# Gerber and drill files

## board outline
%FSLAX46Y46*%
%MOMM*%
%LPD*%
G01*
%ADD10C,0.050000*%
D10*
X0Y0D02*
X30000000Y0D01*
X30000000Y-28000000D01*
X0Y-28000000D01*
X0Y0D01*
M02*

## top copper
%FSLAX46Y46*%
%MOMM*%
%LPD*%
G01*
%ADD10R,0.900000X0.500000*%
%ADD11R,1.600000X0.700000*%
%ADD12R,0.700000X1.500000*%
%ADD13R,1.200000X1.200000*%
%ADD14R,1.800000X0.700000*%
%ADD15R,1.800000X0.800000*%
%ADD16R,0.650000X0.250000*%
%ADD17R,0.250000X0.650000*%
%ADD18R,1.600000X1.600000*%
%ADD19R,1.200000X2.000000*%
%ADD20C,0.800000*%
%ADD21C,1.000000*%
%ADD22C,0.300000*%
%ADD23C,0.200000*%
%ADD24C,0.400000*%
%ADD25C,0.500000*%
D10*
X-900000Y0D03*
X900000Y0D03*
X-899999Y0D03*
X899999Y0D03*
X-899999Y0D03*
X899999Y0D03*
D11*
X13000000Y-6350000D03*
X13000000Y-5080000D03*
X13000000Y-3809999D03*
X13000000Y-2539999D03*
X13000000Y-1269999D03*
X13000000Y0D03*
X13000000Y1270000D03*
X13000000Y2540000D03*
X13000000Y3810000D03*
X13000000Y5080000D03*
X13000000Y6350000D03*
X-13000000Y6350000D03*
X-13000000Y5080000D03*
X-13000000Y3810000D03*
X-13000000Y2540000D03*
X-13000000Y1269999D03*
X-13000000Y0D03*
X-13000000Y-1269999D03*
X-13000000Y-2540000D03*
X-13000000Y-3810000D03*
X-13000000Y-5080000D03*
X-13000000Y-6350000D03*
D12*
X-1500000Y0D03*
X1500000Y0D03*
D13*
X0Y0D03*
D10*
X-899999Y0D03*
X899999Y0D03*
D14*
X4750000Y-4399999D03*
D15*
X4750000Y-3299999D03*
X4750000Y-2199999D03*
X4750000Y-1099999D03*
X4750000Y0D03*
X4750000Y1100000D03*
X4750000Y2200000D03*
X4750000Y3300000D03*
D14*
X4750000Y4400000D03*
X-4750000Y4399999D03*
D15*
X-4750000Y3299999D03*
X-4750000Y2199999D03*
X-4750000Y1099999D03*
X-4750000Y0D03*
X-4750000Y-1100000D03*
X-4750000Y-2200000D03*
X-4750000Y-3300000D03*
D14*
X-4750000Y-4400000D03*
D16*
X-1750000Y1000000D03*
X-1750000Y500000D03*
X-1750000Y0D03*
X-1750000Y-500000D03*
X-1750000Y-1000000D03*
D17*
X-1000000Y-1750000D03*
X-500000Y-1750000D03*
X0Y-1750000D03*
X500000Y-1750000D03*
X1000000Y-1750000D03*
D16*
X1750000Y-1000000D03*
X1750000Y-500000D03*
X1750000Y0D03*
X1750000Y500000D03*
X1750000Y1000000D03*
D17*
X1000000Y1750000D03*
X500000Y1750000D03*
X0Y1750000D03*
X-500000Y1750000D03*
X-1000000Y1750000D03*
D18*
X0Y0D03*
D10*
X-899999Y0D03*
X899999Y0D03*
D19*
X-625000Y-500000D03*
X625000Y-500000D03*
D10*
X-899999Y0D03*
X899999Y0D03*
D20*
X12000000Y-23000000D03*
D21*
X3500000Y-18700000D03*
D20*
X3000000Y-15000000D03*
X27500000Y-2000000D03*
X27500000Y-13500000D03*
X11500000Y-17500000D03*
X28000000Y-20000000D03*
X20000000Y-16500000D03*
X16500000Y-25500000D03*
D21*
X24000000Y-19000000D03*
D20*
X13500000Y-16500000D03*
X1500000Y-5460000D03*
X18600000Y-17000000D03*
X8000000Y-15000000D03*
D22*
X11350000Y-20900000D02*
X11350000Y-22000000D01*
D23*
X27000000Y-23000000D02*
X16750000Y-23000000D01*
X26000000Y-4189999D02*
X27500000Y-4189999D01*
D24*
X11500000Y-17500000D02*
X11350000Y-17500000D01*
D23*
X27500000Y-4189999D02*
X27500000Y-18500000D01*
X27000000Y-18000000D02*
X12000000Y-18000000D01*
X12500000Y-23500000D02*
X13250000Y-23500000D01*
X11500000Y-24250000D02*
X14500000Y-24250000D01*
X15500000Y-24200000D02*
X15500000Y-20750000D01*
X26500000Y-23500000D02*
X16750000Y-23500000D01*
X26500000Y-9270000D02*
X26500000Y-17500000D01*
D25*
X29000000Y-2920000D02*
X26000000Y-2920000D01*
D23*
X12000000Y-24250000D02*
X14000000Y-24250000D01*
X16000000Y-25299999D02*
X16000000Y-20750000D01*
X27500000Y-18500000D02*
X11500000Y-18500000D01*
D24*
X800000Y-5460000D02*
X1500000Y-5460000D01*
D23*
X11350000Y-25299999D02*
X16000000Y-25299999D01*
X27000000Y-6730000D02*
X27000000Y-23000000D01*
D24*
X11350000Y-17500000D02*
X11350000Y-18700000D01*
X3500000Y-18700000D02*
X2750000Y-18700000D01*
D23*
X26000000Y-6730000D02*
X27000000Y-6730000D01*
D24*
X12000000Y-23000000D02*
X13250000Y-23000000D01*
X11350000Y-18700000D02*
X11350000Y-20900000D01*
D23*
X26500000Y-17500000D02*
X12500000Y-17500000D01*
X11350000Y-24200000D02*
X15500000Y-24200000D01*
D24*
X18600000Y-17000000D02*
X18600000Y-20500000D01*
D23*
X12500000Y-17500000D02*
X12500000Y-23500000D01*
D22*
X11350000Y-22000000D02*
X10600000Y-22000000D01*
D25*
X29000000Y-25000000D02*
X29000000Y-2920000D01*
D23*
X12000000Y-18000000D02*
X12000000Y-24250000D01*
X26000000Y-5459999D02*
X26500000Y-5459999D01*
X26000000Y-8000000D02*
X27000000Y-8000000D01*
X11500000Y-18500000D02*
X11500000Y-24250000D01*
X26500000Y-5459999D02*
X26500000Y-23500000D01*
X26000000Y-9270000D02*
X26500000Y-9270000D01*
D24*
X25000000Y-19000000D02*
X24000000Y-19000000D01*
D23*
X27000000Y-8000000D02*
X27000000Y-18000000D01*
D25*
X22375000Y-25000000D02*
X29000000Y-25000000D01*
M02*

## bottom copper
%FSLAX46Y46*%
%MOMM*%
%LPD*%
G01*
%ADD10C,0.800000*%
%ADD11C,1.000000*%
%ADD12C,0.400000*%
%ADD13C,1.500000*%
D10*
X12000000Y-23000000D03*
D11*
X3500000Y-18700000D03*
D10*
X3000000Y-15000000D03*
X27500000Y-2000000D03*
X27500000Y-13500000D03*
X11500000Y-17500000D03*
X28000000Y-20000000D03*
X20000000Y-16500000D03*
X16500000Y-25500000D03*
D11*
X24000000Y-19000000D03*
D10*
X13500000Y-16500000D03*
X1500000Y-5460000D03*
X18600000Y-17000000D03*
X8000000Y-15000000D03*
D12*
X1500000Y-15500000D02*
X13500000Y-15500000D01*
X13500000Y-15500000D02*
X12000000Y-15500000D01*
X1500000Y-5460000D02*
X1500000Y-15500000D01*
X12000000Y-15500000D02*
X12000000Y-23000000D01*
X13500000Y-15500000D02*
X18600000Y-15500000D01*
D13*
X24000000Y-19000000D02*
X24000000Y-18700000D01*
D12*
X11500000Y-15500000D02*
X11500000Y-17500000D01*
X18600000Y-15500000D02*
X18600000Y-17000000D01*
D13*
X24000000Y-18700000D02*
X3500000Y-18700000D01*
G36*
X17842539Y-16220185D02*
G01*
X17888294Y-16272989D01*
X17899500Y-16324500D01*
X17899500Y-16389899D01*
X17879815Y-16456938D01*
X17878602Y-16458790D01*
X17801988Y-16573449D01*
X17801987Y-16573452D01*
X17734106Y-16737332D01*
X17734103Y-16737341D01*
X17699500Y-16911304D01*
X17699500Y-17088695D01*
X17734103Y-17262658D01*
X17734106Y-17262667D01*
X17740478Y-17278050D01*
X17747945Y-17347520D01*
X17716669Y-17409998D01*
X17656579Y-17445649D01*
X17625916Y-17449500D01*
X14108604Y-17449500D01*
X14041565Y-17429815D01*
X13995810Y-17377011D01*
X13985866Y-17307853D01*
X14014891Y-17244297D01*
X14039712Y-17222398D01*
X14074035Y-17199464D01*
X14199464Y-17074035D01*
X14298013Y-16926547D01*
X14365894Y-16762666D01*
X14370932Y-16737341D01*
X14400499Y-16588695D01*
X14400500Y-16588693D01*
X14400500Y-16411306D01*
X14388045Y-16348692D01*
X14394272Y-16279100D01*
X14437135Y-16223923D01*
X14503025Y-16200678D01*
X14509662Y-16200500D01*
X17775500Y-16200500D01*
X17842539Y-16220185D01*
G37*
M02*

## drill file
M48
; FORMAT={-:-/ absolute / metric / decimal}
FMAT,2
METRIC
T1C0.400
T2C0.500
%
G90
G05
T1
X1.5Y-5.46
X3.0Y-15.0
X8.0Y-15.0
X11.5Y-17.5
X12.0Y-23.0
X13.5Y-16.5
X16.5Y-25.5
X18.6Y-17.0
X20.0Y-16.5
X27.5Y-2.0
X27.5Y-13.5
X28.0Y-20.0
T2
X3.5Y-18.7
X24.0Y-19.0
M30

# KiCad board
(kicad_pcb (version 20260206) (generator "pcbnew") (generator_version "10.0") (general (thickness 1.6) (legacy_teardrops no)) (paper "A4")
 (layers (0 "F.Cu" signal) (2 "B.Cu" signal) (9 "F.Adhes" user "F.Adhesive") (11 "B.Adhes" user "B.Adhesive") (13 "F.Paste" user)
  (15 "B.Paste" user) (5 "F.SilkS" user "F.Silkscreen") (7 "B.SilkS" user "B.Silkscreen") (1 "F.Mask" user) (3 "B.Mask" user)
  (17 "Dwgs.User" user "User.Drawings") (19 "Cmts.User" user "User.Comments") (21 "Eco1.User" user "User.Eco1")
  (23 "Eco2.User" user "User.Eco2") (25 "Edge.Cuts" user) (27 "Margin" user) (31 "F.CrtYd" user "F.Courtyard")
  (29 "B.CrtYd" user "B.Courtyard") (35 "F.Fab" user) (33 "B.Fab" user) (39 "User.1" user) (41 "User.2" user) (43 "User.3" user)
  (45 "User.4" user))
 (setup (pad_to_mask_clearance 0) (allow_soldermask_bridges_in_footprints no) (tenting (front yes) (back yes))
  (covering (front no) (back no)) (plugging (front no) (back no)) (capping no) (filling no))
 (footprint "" (layer "F.Cu") (at 11.5 22)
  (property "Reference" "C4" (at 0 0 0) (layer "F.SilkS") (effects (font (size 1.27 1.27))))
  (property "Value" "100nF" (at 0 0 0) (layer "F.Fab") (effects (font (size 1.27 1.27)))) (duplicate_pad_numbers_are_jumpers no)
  (pad "1" smd rect (at -12.4 -22) (size 0.9 0.5) (layers "F.Cu" "F.Mask" "F.Paste") (thermal_bridge_angle 45))
  (pad "2" smd rect (at -10.6 -22) (size 0.9 0.5) (layers "F.Cu" "F.Mask" "F.Paste") (thermal_bridge_angle 45)))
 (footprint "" (layer "F.Cu") (at 27.5 5.5)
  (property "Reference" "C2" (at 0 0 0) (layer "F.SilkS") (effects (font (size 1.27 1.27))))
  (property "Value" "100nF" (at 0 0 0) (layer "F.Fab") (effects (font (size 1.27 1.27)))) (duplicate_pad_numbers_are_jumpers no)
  (pad "1" smd rect (at -28.399999 -5.5) (size 0.9 0.5) (layers "F.Cu" "F.Mask" "F.Paste") (thermal_bridge_angle 45))
  (pad "2" smd rect (at -26.600001 -5.5) (size 0.9 0.5) (layers "F.Cu" "F.Mask" "F.Paste") (thermal_bridge_angle 45)))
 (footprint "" (layer "F.Cu") (at 27.5 2.5)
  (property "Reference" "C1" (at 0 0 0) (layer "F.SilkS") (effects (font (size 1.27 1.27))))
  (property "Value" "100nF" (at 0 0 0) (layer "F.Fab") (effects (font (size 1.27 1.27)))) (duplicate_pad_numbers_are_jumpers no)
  (pad "1" smd rect (at -28.399999 -2.5) (size 0.9 0.5) (layers "F.Cu" "F.Mask" "F.Paste") (thermal_bridge_angle 45))
  (pad "2" smd rect (at -26.600001 -2.5) (size 0.9 0.5) (layers "F.Cu" "F.Mask" "F.Paste") (thermal_bridge_angle 45)))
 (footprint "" (layer "F.Cu") (at 13 8)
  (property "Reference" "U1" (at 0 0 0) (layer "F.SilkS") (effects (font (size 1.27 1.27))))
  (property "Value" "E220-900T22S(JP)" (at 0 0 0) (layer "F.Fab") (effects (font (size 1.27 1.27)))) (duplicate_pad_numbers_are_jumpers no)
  (pad "1" smd rect (at 0 -1.65) (size 1.6 0.7) (layers "F.Cu" "F.Mask" "F.Paste") (thermal_bridge_angle 45))
  (pad "2" smd rect (at 0 -2.92) (size 1.6 0.7) (layers "F.Cu" "F.Mask" "F.Paste") (thermal_bridge_angle 45))
  (pad "3" smd rect (at 0 -4.190001) (size 1.6 0.7) (layers "F.Cu" "F.Mask" "F.Paste") (thermal_bridge_angle 45))
  (pad "4" smd rect (at 0 -5.460001) (size 1.6 0.7) (layers "F.Cu" "F.Mask" "F.Paste") (thermal_bridge_angle 45))
  (pad "5" smd rect (at 0 -6.730001) (size 1.6 0.7) (layers "F.Cu" "F.Mask" "F.Paste") (thermal_bridge_angle 45))
  (pad "6" smd rect (at 0 -8) (size 1.6 0.7) (layers "F.Cu" "F.Mask" "F.Paste") (thermal_bridge_angle 45))
  (pad "7" smd rect (at 0 -9.27) (size 1.6 0.7) (layers "F.Cu" "F.Mask" "F.Paste") (thermal_bridge_angle 45))
  (pad "8" smd rect (at 0 -10.54) (size 1.6 0.7) (layers "F.Cu" "F.Mask" "F.Paste") (thermal_bridge_angle 45))
  (pad "9" smd rect (at 0 -11.81) (size 1.6 0.7) (layers "F.Cu" "F.Mask" "F.Paste") (thermal_bridge_angle 45))
  (pad "10" smd rect (at 0 -13.08) (size 1.6 0.7) (layers "F.Cu" "F.Mask" "F.Paste") (thermal_bridge_angle 45))
  (pad "11" smd rect (at 0 -14.35) (size 1.6 0.7) (layers "F.Cu" "F.Mask" "F.Paste") (thermal_bridge_angle 45))
  (pad "12" smd rect (at -26 -14.35) (size 1.6 0.7) (layers "F.Cu" "F.Mask" "F.Paste") (thermal_bridge_angle 45))
  (pad "13" smd rect (at -26 -13.08) (size 1.6 0.7) (layers "F.Cu" "F.Mask" "F.Paste") (thermal_bridge_angle 45))
  (pad "14" smd rect (at -26 -11.81) (size 1.6 0.7) (layers "F.Cu" "F.Mask" "F.Paste") (thermal_bridge_angle 45))
  (pad "15" smd rect (at -26 -10.54) (size 1.6 0.7) (layers "F.Cu" "F.Mask" "F.Paste") (thermal_bridge_angle 45))
  (pad "16" smd rect (at -26 -9.269999) (size 1.6 0.7) (layers "F.Cu" "F.Mask" "F.Paste") (thermal_bridge_angle 45))
  (pad "17" smd rect (at -26 -8) (size 1.6 0.7) (layers "F.Cu" "F.Mask" "F.Paste") (thermal_bridge_angle 45))
  (pad "18" smd rect (at -26 -6.730001) (size 1.6 0.7) (layers "F.Cu" "F.Mask" "F.Paste") (thermal_bridge_angle 45))
  (pad "19" smd rect (at -26 -5.46) (size 1.6 0.7) (layers "F.Cu" "F.Mask" "F.Paste") (thermal_bridge_angle 45))
  (pad "20" smd rect (at -26 -4.19) (size 1.6 0.7) (layers "F.Cu" "F.Mask" "F.Paste") (thermal_bridge_angle 45))
  (pad "21" smd rect (at -26 -2.92) (size 1.6 0.7) (layers "F.Cu" "F.Mask" "F.Paste") (thermal_bridge_angle 45))
  (pad "22" smd rect (at -26 -1.65) (size 1.6 0.7) (layers "F.Cu" "F.Mask" "F.Paste") (thermal_bridge_angle 45)))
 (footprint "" (layer "F.Cu") (at 25 19)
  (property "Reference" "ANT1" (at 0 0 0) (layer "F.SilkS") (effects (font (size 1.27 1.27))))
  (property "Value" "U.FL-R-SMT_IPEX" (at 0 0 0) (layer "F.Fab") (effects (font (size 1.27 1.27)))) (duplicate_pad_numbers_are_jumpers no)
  (pad "G1" smd rect (at -26.5 -19) (size 0.7 1.5) (layers "F.Cu" "F.Mask" "F.Paste") (thermal_bridge_angle 45))
  (pad "G2" smd rect (at -23.5 -19) (size 0.7 1.5) (layers "F.Cu" "F.Mask" "F.Paste") (thermal_bridge_angle 45))
  (pad "S" smd rect (at -25 -19) (size 1.2 1.2) (layers "F.Cu" "F.Mask" "F.Paste") (thermal_bridge_angle 45)))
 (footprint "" (layer "F.Cu") (at 19.5 24.5)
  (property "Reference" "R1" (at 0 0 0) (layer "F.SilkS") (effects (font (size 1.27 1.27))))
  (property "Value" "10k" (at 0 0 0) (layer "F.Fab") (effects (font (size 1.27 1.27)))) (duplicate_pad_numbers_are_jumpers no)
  (pad "1" smd rect (at -20.399999 -24.5) (size 0.9 0.5) (layers "F.Cu" "F.Mask" "F.Paste") (thermal_bridge_angle 45))
  (pad "2" smd rect (at -18.600001 -24.5) (size 0.9 0.5) (layers "F.Cu" "F.Mask" "F.Paste") (thermal_bridge_angle 45)))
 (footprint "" (layer "F.Cu") (at 6.6 22)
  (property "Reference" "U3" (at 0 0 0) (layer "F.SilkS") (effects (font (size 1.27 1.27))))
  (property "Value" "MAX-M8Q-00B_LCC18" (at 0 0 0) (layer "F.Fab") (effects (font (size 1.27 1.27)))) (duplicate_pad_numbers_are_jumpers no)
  (pad "1" smd rect (at -1.85 -17.600001) (size 1.8 0.7) (layers "F.Cu" "F.Mask" "F.Paste") (thermal_bridge_angle 45))
  (pad "2" smd rect (at -1.85 -18.700001) (size 1.8 0.8) (layers "F.Cu" "F.Mask" "F.Paste") (thermal_bridge_angle 45))
  (pad "3" smd rect (at -1.85 -19.800001) (size 1.8 0.8) (layers "F.Cu" "F.Mask" "F.Paste") (thermal_bridge_angle 45))
  (pad "4" smd rect (at -1.85 -20.900001) (size 1.8 0.8) (layers "F.Cu" "F.Mask" "F.Paste") (thermal_bridge_angle 45))
  (pad "5" smd rect (at -1.85 -22) (size 1.8 0.8) (layers "F.Cu" "F.Mask" "F.Paste") (thermal_bridge_angle 45))
  (pad "6" smd rect (at -1.85 -23.1) (size 1.8 0.8) (layers "F.Cu" "F.Mask" "F.Paste") (thermal_bridge_angle 45))
  (pad "7" smd rect (at -1.85 -24.2) (size 1.8 0.8) (layers "F.Cu" "F.Mask" "F.Paste") (thermal_bridge_angle 45))
  (pad "8" smd rect (at -1.85 -25.3) (size 1.8 0.8) (layers "F.Cu" "F.Mask" "F.Paste") (thermal_bridge_angle 45))
  (pad "9" smd rect (at -1.85 -26.4) (size 1.8 0.7) (layers "F.Cu" "F.Mask" "F.Paste") (thermal_bridge_angle 45))
  (pad "10" smd rect (at -11.35 -26.399999) (size 1.8 0.7) (layers "F.Cu" "F.Mask" "F.Paste") (thermal_bridge_angle 45))
  (pad "11" smd rect (at -11.35 -25.299999) (size 1.8 0.8) (layers "F.Cu" "F.Mask" "F.Paste") (thermal_bridge_angle 45))
  (pad "12" smd rect (at -11.35 -24.199999) (size 1.8 0.8) (layers "F.Cu" "F.Mask" "F.Paste") (thermal_bridge_angle 45))
  (pad "13" smd rect (at -11.35 -23.099999) (size 1.8 0.8) (layers "F.Cu" "F.Mask" "F.Paste") (thermal_bridge_angle 45))
  (pad "14" smd rect (at -11.35 -22) (size 1.8 0.8) (layers "F.Cu" "F.Mask" "F.Paste") (thermal_bridge_angle 45))
  (pad "15" smd rect (at -11.35 -20.9) (size 1.8 0.8) (layers "F.Cu" "F.Mask" "F.Paste") (thermal_bridge_angle 45))
  (pad "16" smd rect (at -11.35 -19.8) (size 1.8 0.8) (layers "F.Cu" "F.Mask" "F.Paste") (thermal_bridge_angle 45))
  (pad "17" smd rect (at -11.35 -18.7) (size 1.8 0.8) (layers "F.Cu" "F.Mask" "F.Paste") (thermal_bridge_angle 45))
  (pad "18" smd rect (at -11.35 -17.6) (size 1.8 0.7) (layers "F.Cu" "F.Mask" "F.Paste") (thermal_bridge_angle 45)))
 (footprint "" (layer "F.Cu") (at 15 22.5)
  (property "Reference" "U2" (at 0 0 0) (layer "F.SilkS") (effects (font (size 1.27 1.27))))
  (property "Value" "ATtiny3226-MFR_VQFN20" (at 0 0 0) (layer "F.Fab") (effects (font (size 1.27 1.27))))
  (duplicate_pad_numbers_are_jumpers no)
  (pad "1" smd rect (at -16.75 -23.5) (size 0.65 0.25) (layers "F.Cu" "F.Mask" "F.Paste") (thermal_bridge_angle 45))
  (pad "2" smd rect (at -16.75 -23) (size 0.65 0.25) (layers "F.Cu" "F.Mask" "F.Paste") (thermal_bridge_angle 45))
  (pad "3" smd rect (at -16.75 -22.5) (size 0.65 0.25) (layers "F.Cu" "F.Mask" "F.Paste") (thermal_bridge_angle 45))
  (pad "4" smd rect (at -16.75 -22) (size 0.65 0.25) (layers "F.Cu" "F.Mask" "F.Paste") (thermal_bridge_angle 45))
  (pad "5" smd rect (at -16.75 -21.5) (size 0.65 0.25) (layers "F.Cu" "F.Mask" "F.Paste") (thermal_bridge_angle 45))
  (pad "6" smd rect (at -16 -20.75) (size 0.25 0.65) (layers "F.Cu" "F.Mask" "F.Paste") (thermal_bridge_angle 45))
  (pad "7" smd rect (at -15.5 -20.75) (size 0.25 0.65) (layers "F.Cu" "F.Mask" "F.Paste") (thermal_bridge_angle 45))
  (pad "8" smd rect (at -15 -20.75) (size 0.25 0.65) (layers "F.Cu" "F.Mask" "F.Paste") (thermal_bridge_angle 45))
  (pad "9" smd rect (at -14.5 -20.75) (size 0.25 0.65) (layers "F.Cu" "F.Mask" "F.Paste") (thermal_bridge_angle 45))
  (pad "10" smd rect (at -14 -20.75) (size 0.25 0.65) (layers "F.Cu" "F.Mask" "F.Paste") (thermal_bridge_angle 45))
  (pad "11" smd rect (at -13.25 -21.5) (size 0.65 0.25) (layers "F.Cu" "F.Mask" "F.Paste") (thermal_bridge_angle 45))
  (pad "12" smd rect (at -13.25 -22) (size 0.65 0.25) (layers "F.Cu" "F.Mask" "F.Paste") (thermal_bridge_angle 45))
  (pad "13" smd rect (at -13.25 -22.5) (size 0.65 0.25) (layers "F.Cu" "F.Mask" "F.Paste") (thermal_bridge_angle 45))
  (pad "14" smd rect (at -13.25 -23) (size 0.65 0.25) (layers "F.Cu" "F.Mask" "F.Paste") (thermal_bridge_angle 45))
  (pad "15" smd rect (at -13.25 -23.5) (size 0.65 0.25) (layers "F.Cu" "F.Mask" "F.Paste") (thermal_bridge_angle 45))
  (pad "16" smd rect (at -14 -24.25) (size 0.25 0.65) (layers "F.Cu" "F.Mask" "F.Paste") (thermal_bridge_angle 45))
  (pad "17" smd rect (at -14.5 -24.25) (size 0.25 0.65) (layers "F.Cu" "F.Mask" "F.Paste") (thermal_bridge_angle 45))
  (pad "18" smd rect (at -15 -24.25) (size 0.25 0.65) (layers "F.Cu" "F.Mask" "F.Paste") (thermal_bridge_angle 45))
  (pad "19" smd rect (at -15.5 -24.25) (size 0.25 0.65) (layers "F.Cu" "F.Mask" "F.Paste") (thermal_bridge_angle 45))
  (pad "20" smd rect (at -16 -24.25) (size 0.25 0.65) (layers "F.Cu" "F.Mask" "F.Paste") (thermal_bridge_angle 45))
  (pad "EP" smd rect (at -15 -22.5) (size 1.6 1.6) (layers "F.Cu" "F.Mask" "F.Paste") (thermal_bridge_angle 45)))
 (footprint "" (layer "F.Cu") (at 27.5 8.5)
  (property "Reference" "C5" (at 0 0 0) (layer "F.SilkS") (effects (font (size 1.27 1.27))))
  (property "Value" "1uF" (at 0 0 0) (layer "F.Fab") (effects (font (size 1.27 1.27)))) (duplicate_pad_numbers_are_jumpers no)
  (pad "1" smd rect (at -28.399999 -8.5) (size 0.9 0.5) (layers "F.Cu" "F.Mask" "F.Paste") (thermal_bridge_angle 45))
  (pad "2" smd rect (at -26.600001 -8.5) (size 0.9 0.5) (layers "F.Cu" "F.Mask" "F.Paste") (thermal_bridge_angle 45)))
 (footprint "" (layer "F.Cu") (at 23 24.5)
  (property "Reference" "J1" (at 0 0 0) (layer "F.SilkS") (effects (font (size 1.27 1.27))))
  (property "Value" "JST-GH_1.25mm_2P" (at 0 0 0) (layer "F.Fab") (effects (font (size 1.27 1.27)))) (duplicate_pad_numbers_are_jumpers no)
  (pad "1" smd rect (at -23.625 -24) (size 1.2 2) (layers "F.Cu" "F.Mask" "F.Paste") (thermal_bridge_angle 45))
  (pad "2" smd rect (at -22.375 -24) (size 1.2 2) (layers "F.Cu" "F.Mask" "F.Paste") (thermal_bridge_angle 45)))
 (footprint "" (layer "F.Cu") (at 19.5 20.5)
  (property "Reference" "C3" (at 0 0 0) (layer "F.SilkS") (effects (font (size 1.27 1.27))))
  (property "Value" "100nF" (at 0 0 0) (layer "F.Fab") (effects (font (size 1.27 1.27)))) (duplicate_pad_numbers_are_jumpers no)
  (pad "1" smd rect (at -20.399999 -20.5) (size 0.9 0.5) (layers "F.Cu" "F.Mask" "F.Paste") (thermal_bridge_angle 45))
  (pad "2" smd rect (at -18.600001 -20.5) (size 0.9 0.5) (layers "F.Cu" "F.Mask" "F.Paste") (thermal_bridge_angle 45)))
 (gr_rect (start 0 0) (end 30 28) (stroke (width 0.05) (type default)) (fill no) (layer "Edge.Cuts"))
 (segment (start 11.35 20.9) (end 11.35 22) (width 0.3) (layer "F.Cu") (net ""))
 (segment (start 27 23) (end 16.75 23) (width 0.2) (layer "F.Cu") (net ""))
 (segment (start 26 4.189999) (end 27.5 4.189999) (width 0.2) (layer "F.Cu") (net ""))
 (segment (start 11.5 17.5) (end 11.35 17.5) (width 0.4) (layer "F.Cu") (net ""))
 (segment (start 27.5 4.189999) (end 27.5 18.5) (width 0.2) (layer "F.Cu") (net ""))
 (segment (start 27 18) (end 12 18) (width 0.2) (layer "F.Cu") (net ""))
 (segment (start 12.5 23.5) (end 13.25 23.5) (width 0.2) (layer "F.Cu") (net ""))
 (segment (start 11.5 24.25) (end 14.5 24.25) (width 0.2) (layer "F.Cu") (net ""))
 (segment (start 15.5 24.2) (end 15.5 20.75) (width 0.2) (layer "F.Cu") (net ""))
 (segment (start 26.5 23.5) (end 16.75 23.5) (width 0.2) (layer "F.Cu") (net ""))
 (segment (start 26.5 9.27) (end 26.5 17.5) (width 0.2) (layer "F.Cu") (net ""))
 (segment (start 29 2.92) (end 26 2.92) (width 0.5) (layer "F.Cu") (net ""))
 (segment (start 12 24.25) (end 14 24.25) (width 0.2) (layer "F.Cu") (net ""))
 (segment (start 16 25.299999) (end 16 20.75) (width 0.2) (layer "F.Cu") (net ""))
 (segment (start 27.5 18.5) (end 11.5 18.5) (width 0.2) (layer "F.Cu") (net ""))
 (segment (start 0.8 5.46) (end 1.5 5.46) (width 0.4) (layer "F.Cu") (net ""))
 (segment (start 11.35 25.299999) (end 16 25.299999) (width 0.2) (layer "F.Cu") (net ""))
 (segment (start 27 6.73) (end 27 23) (width 0.2) (layer "F.Cu") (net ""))
 (segment (start 11.35 17.5) (end 11.35 18.7) (width 0.4) (layer "F.Cu") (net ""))
 (segment (start 3.5 18.7) (end 2.75 18.7) (width 0.4) (layer "F.Cu") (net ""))
 (segment (start 26 6.73) (end 27 6.73) (width 0.2) (layer "F.Cu") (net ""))
 (segment (start 12 23) (end 13.25 23) (width 0.4) (layer "F.Cu") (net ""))
 (segment (start 11.35 18.7) (end 11.35 20.9) (width 0.4) (layer "F.Cu") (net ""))
 (segment (start 26.5 17.5) (end 12.5 17.5) (width 0.2) (layer "F.Cu") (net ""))
 (segment (start 11.35 24.2) (end 15.5 24.2) (width 0.2) (layer "F.Cu") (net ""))
 (segment (start 18.6 17) (end 18.6 20.5) (width 0.4) (layer "F.Cu") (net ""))
 (segment (start 12.5 17.5) (end 12.5 23.5) (width 0.2) (layer "F.Cu") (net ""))
 (segment (start 11.35 22) (end 10.6 22) (width 0.3) (layer "F.Cu") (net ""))
 (segment (start 29 25) (end 29 2.92) (width 0.5) (layer "F.Cu") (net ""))
 (segment (start 12 18) (end 12 24.25) (width 0.2) (layer "F.Cu") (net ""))
 (segment (start 26 5.459999) (end 26.5 5.459999) (width 0.2) (layer "F.Cu") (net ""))
 (segment (start 26 8) (end 27 8) (width 0.2) (layer "F.Cu") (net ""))
 (segment (start 11.5 18.5) (end 11.5 24.25) (width 0.2) (layer "F.Cu") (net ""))
 (segment (start 26.5 5.459999) (end 26.5 23.5) (width 0.2) (layer "F.Cu") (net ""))
 (segment (start 26 9.27) (end 26.5 9.27) (width 0.2) (layer "F.Cu") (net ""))
 (segment (start 25 19) (end 24 19) (width 0.4) (layer "F.Cu") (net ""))
 (segment (start 27 8) (end 27 18) (width 0.2) (layer "F.Cu") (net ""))
 (segment (start 22.375 25) (end 29 25) (width 0.5) (layer "F.Cu") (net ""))
 (via (at 12 23) (size 0.8) (drill 0.4) (layers "F.Cu" "B.Cu") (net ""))
 (via (at 3.5 18.7) (size 1) (drill 0.5) (layers "F.Cu" "B.Cu") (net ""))
 (via (at 3 15) (size 0.8) (drill 0.4) (layers "F.Cu" "B.Cu") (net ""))
 (via (at 27.5 2) (size 0.8) (drill 0.4) (layers "F.Cu" "B.Cu") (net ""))
 (via (at 27.5 13.5) (size 0.8) (drill 0.4) (layers "F.Cu" "B.Cu") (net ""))
 (via (at 11.5 17.5) (size 0.8) (drill 0.4) (layers "F.Cu" "B.Cu") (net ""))
 (via (at 28 20) (size 0.8) (drill 0.4) (layers "F.Cu" "B.Cu") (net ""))
 (via (at 20 16.5) (size 0.8) (drill 0.4) (layers "F.Cu" "B.Cu") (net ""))
 (via (at 16.5 25.5) (size 0.8) (drill 0.4) (layers "F.Cu" "B.Cu") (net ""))
 (via (at 24 19) (size 1) (drill 0.5) (layers "F.Cu" "B.Cu") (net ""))
 (via (at 13.5 16.5) (size 0.8) (drill 0.4) (layers "F.Cu" "B.Cu") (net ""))
 (via (at 1.5 5.46) (size 0.8) (drill 0.4) (layers "F.Cu" "B.Cu") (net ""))
 (via (at 18.6 17) (size 0.8) (drill 0.4) (layers "F.Cu" "B.Cu") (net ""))
 (via (at 8 15) (size 0.8) (drill 0.4) (layers "F.Cu" "B.Cu") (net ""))
 (segment (start 1.5 15.5) (end 13.5 15.5) (width 0.4) (layer "B.Cu") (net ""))
 (segment (start 13.5 15.5) (end 12 15.5) (width 0.4) (layer "B.Cu") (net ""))
 (segment (start 1.5 5.46) (end 1.5 15.5) (width 0.4) (layer "B.Cu") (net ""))
 (segment (start 12 15.5) (end 12 23) (width 0.4) (layer "B.Cu") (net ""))
 (segment (start 13.5 15.5) (end 18.6 15.5) (width 0.4) (layer "B.Cu") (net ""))
 (segment (start 24 19) (end 24 18.7) (width 1.5) (layer "B.Cu") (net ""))
 (segment (start 11.5 15.5) (end 11.5 17.5) (width 0.4) (layer "B.Cu") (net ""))
 (segment (start 18.6 15.5) (end 18.6 17) (width 0.4) (layer "B.Cu") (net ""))
 (segment (start 24 18.7) (end 3.5 18.7) (width 1.5) (layer "B.Cu") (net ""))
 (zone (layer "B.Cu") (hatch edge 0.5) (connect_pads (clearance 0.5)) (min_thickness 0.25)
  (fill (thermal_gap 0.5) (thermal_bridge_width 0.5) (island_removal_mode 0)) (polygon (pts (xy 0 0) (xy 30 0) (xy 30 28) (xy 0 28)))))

